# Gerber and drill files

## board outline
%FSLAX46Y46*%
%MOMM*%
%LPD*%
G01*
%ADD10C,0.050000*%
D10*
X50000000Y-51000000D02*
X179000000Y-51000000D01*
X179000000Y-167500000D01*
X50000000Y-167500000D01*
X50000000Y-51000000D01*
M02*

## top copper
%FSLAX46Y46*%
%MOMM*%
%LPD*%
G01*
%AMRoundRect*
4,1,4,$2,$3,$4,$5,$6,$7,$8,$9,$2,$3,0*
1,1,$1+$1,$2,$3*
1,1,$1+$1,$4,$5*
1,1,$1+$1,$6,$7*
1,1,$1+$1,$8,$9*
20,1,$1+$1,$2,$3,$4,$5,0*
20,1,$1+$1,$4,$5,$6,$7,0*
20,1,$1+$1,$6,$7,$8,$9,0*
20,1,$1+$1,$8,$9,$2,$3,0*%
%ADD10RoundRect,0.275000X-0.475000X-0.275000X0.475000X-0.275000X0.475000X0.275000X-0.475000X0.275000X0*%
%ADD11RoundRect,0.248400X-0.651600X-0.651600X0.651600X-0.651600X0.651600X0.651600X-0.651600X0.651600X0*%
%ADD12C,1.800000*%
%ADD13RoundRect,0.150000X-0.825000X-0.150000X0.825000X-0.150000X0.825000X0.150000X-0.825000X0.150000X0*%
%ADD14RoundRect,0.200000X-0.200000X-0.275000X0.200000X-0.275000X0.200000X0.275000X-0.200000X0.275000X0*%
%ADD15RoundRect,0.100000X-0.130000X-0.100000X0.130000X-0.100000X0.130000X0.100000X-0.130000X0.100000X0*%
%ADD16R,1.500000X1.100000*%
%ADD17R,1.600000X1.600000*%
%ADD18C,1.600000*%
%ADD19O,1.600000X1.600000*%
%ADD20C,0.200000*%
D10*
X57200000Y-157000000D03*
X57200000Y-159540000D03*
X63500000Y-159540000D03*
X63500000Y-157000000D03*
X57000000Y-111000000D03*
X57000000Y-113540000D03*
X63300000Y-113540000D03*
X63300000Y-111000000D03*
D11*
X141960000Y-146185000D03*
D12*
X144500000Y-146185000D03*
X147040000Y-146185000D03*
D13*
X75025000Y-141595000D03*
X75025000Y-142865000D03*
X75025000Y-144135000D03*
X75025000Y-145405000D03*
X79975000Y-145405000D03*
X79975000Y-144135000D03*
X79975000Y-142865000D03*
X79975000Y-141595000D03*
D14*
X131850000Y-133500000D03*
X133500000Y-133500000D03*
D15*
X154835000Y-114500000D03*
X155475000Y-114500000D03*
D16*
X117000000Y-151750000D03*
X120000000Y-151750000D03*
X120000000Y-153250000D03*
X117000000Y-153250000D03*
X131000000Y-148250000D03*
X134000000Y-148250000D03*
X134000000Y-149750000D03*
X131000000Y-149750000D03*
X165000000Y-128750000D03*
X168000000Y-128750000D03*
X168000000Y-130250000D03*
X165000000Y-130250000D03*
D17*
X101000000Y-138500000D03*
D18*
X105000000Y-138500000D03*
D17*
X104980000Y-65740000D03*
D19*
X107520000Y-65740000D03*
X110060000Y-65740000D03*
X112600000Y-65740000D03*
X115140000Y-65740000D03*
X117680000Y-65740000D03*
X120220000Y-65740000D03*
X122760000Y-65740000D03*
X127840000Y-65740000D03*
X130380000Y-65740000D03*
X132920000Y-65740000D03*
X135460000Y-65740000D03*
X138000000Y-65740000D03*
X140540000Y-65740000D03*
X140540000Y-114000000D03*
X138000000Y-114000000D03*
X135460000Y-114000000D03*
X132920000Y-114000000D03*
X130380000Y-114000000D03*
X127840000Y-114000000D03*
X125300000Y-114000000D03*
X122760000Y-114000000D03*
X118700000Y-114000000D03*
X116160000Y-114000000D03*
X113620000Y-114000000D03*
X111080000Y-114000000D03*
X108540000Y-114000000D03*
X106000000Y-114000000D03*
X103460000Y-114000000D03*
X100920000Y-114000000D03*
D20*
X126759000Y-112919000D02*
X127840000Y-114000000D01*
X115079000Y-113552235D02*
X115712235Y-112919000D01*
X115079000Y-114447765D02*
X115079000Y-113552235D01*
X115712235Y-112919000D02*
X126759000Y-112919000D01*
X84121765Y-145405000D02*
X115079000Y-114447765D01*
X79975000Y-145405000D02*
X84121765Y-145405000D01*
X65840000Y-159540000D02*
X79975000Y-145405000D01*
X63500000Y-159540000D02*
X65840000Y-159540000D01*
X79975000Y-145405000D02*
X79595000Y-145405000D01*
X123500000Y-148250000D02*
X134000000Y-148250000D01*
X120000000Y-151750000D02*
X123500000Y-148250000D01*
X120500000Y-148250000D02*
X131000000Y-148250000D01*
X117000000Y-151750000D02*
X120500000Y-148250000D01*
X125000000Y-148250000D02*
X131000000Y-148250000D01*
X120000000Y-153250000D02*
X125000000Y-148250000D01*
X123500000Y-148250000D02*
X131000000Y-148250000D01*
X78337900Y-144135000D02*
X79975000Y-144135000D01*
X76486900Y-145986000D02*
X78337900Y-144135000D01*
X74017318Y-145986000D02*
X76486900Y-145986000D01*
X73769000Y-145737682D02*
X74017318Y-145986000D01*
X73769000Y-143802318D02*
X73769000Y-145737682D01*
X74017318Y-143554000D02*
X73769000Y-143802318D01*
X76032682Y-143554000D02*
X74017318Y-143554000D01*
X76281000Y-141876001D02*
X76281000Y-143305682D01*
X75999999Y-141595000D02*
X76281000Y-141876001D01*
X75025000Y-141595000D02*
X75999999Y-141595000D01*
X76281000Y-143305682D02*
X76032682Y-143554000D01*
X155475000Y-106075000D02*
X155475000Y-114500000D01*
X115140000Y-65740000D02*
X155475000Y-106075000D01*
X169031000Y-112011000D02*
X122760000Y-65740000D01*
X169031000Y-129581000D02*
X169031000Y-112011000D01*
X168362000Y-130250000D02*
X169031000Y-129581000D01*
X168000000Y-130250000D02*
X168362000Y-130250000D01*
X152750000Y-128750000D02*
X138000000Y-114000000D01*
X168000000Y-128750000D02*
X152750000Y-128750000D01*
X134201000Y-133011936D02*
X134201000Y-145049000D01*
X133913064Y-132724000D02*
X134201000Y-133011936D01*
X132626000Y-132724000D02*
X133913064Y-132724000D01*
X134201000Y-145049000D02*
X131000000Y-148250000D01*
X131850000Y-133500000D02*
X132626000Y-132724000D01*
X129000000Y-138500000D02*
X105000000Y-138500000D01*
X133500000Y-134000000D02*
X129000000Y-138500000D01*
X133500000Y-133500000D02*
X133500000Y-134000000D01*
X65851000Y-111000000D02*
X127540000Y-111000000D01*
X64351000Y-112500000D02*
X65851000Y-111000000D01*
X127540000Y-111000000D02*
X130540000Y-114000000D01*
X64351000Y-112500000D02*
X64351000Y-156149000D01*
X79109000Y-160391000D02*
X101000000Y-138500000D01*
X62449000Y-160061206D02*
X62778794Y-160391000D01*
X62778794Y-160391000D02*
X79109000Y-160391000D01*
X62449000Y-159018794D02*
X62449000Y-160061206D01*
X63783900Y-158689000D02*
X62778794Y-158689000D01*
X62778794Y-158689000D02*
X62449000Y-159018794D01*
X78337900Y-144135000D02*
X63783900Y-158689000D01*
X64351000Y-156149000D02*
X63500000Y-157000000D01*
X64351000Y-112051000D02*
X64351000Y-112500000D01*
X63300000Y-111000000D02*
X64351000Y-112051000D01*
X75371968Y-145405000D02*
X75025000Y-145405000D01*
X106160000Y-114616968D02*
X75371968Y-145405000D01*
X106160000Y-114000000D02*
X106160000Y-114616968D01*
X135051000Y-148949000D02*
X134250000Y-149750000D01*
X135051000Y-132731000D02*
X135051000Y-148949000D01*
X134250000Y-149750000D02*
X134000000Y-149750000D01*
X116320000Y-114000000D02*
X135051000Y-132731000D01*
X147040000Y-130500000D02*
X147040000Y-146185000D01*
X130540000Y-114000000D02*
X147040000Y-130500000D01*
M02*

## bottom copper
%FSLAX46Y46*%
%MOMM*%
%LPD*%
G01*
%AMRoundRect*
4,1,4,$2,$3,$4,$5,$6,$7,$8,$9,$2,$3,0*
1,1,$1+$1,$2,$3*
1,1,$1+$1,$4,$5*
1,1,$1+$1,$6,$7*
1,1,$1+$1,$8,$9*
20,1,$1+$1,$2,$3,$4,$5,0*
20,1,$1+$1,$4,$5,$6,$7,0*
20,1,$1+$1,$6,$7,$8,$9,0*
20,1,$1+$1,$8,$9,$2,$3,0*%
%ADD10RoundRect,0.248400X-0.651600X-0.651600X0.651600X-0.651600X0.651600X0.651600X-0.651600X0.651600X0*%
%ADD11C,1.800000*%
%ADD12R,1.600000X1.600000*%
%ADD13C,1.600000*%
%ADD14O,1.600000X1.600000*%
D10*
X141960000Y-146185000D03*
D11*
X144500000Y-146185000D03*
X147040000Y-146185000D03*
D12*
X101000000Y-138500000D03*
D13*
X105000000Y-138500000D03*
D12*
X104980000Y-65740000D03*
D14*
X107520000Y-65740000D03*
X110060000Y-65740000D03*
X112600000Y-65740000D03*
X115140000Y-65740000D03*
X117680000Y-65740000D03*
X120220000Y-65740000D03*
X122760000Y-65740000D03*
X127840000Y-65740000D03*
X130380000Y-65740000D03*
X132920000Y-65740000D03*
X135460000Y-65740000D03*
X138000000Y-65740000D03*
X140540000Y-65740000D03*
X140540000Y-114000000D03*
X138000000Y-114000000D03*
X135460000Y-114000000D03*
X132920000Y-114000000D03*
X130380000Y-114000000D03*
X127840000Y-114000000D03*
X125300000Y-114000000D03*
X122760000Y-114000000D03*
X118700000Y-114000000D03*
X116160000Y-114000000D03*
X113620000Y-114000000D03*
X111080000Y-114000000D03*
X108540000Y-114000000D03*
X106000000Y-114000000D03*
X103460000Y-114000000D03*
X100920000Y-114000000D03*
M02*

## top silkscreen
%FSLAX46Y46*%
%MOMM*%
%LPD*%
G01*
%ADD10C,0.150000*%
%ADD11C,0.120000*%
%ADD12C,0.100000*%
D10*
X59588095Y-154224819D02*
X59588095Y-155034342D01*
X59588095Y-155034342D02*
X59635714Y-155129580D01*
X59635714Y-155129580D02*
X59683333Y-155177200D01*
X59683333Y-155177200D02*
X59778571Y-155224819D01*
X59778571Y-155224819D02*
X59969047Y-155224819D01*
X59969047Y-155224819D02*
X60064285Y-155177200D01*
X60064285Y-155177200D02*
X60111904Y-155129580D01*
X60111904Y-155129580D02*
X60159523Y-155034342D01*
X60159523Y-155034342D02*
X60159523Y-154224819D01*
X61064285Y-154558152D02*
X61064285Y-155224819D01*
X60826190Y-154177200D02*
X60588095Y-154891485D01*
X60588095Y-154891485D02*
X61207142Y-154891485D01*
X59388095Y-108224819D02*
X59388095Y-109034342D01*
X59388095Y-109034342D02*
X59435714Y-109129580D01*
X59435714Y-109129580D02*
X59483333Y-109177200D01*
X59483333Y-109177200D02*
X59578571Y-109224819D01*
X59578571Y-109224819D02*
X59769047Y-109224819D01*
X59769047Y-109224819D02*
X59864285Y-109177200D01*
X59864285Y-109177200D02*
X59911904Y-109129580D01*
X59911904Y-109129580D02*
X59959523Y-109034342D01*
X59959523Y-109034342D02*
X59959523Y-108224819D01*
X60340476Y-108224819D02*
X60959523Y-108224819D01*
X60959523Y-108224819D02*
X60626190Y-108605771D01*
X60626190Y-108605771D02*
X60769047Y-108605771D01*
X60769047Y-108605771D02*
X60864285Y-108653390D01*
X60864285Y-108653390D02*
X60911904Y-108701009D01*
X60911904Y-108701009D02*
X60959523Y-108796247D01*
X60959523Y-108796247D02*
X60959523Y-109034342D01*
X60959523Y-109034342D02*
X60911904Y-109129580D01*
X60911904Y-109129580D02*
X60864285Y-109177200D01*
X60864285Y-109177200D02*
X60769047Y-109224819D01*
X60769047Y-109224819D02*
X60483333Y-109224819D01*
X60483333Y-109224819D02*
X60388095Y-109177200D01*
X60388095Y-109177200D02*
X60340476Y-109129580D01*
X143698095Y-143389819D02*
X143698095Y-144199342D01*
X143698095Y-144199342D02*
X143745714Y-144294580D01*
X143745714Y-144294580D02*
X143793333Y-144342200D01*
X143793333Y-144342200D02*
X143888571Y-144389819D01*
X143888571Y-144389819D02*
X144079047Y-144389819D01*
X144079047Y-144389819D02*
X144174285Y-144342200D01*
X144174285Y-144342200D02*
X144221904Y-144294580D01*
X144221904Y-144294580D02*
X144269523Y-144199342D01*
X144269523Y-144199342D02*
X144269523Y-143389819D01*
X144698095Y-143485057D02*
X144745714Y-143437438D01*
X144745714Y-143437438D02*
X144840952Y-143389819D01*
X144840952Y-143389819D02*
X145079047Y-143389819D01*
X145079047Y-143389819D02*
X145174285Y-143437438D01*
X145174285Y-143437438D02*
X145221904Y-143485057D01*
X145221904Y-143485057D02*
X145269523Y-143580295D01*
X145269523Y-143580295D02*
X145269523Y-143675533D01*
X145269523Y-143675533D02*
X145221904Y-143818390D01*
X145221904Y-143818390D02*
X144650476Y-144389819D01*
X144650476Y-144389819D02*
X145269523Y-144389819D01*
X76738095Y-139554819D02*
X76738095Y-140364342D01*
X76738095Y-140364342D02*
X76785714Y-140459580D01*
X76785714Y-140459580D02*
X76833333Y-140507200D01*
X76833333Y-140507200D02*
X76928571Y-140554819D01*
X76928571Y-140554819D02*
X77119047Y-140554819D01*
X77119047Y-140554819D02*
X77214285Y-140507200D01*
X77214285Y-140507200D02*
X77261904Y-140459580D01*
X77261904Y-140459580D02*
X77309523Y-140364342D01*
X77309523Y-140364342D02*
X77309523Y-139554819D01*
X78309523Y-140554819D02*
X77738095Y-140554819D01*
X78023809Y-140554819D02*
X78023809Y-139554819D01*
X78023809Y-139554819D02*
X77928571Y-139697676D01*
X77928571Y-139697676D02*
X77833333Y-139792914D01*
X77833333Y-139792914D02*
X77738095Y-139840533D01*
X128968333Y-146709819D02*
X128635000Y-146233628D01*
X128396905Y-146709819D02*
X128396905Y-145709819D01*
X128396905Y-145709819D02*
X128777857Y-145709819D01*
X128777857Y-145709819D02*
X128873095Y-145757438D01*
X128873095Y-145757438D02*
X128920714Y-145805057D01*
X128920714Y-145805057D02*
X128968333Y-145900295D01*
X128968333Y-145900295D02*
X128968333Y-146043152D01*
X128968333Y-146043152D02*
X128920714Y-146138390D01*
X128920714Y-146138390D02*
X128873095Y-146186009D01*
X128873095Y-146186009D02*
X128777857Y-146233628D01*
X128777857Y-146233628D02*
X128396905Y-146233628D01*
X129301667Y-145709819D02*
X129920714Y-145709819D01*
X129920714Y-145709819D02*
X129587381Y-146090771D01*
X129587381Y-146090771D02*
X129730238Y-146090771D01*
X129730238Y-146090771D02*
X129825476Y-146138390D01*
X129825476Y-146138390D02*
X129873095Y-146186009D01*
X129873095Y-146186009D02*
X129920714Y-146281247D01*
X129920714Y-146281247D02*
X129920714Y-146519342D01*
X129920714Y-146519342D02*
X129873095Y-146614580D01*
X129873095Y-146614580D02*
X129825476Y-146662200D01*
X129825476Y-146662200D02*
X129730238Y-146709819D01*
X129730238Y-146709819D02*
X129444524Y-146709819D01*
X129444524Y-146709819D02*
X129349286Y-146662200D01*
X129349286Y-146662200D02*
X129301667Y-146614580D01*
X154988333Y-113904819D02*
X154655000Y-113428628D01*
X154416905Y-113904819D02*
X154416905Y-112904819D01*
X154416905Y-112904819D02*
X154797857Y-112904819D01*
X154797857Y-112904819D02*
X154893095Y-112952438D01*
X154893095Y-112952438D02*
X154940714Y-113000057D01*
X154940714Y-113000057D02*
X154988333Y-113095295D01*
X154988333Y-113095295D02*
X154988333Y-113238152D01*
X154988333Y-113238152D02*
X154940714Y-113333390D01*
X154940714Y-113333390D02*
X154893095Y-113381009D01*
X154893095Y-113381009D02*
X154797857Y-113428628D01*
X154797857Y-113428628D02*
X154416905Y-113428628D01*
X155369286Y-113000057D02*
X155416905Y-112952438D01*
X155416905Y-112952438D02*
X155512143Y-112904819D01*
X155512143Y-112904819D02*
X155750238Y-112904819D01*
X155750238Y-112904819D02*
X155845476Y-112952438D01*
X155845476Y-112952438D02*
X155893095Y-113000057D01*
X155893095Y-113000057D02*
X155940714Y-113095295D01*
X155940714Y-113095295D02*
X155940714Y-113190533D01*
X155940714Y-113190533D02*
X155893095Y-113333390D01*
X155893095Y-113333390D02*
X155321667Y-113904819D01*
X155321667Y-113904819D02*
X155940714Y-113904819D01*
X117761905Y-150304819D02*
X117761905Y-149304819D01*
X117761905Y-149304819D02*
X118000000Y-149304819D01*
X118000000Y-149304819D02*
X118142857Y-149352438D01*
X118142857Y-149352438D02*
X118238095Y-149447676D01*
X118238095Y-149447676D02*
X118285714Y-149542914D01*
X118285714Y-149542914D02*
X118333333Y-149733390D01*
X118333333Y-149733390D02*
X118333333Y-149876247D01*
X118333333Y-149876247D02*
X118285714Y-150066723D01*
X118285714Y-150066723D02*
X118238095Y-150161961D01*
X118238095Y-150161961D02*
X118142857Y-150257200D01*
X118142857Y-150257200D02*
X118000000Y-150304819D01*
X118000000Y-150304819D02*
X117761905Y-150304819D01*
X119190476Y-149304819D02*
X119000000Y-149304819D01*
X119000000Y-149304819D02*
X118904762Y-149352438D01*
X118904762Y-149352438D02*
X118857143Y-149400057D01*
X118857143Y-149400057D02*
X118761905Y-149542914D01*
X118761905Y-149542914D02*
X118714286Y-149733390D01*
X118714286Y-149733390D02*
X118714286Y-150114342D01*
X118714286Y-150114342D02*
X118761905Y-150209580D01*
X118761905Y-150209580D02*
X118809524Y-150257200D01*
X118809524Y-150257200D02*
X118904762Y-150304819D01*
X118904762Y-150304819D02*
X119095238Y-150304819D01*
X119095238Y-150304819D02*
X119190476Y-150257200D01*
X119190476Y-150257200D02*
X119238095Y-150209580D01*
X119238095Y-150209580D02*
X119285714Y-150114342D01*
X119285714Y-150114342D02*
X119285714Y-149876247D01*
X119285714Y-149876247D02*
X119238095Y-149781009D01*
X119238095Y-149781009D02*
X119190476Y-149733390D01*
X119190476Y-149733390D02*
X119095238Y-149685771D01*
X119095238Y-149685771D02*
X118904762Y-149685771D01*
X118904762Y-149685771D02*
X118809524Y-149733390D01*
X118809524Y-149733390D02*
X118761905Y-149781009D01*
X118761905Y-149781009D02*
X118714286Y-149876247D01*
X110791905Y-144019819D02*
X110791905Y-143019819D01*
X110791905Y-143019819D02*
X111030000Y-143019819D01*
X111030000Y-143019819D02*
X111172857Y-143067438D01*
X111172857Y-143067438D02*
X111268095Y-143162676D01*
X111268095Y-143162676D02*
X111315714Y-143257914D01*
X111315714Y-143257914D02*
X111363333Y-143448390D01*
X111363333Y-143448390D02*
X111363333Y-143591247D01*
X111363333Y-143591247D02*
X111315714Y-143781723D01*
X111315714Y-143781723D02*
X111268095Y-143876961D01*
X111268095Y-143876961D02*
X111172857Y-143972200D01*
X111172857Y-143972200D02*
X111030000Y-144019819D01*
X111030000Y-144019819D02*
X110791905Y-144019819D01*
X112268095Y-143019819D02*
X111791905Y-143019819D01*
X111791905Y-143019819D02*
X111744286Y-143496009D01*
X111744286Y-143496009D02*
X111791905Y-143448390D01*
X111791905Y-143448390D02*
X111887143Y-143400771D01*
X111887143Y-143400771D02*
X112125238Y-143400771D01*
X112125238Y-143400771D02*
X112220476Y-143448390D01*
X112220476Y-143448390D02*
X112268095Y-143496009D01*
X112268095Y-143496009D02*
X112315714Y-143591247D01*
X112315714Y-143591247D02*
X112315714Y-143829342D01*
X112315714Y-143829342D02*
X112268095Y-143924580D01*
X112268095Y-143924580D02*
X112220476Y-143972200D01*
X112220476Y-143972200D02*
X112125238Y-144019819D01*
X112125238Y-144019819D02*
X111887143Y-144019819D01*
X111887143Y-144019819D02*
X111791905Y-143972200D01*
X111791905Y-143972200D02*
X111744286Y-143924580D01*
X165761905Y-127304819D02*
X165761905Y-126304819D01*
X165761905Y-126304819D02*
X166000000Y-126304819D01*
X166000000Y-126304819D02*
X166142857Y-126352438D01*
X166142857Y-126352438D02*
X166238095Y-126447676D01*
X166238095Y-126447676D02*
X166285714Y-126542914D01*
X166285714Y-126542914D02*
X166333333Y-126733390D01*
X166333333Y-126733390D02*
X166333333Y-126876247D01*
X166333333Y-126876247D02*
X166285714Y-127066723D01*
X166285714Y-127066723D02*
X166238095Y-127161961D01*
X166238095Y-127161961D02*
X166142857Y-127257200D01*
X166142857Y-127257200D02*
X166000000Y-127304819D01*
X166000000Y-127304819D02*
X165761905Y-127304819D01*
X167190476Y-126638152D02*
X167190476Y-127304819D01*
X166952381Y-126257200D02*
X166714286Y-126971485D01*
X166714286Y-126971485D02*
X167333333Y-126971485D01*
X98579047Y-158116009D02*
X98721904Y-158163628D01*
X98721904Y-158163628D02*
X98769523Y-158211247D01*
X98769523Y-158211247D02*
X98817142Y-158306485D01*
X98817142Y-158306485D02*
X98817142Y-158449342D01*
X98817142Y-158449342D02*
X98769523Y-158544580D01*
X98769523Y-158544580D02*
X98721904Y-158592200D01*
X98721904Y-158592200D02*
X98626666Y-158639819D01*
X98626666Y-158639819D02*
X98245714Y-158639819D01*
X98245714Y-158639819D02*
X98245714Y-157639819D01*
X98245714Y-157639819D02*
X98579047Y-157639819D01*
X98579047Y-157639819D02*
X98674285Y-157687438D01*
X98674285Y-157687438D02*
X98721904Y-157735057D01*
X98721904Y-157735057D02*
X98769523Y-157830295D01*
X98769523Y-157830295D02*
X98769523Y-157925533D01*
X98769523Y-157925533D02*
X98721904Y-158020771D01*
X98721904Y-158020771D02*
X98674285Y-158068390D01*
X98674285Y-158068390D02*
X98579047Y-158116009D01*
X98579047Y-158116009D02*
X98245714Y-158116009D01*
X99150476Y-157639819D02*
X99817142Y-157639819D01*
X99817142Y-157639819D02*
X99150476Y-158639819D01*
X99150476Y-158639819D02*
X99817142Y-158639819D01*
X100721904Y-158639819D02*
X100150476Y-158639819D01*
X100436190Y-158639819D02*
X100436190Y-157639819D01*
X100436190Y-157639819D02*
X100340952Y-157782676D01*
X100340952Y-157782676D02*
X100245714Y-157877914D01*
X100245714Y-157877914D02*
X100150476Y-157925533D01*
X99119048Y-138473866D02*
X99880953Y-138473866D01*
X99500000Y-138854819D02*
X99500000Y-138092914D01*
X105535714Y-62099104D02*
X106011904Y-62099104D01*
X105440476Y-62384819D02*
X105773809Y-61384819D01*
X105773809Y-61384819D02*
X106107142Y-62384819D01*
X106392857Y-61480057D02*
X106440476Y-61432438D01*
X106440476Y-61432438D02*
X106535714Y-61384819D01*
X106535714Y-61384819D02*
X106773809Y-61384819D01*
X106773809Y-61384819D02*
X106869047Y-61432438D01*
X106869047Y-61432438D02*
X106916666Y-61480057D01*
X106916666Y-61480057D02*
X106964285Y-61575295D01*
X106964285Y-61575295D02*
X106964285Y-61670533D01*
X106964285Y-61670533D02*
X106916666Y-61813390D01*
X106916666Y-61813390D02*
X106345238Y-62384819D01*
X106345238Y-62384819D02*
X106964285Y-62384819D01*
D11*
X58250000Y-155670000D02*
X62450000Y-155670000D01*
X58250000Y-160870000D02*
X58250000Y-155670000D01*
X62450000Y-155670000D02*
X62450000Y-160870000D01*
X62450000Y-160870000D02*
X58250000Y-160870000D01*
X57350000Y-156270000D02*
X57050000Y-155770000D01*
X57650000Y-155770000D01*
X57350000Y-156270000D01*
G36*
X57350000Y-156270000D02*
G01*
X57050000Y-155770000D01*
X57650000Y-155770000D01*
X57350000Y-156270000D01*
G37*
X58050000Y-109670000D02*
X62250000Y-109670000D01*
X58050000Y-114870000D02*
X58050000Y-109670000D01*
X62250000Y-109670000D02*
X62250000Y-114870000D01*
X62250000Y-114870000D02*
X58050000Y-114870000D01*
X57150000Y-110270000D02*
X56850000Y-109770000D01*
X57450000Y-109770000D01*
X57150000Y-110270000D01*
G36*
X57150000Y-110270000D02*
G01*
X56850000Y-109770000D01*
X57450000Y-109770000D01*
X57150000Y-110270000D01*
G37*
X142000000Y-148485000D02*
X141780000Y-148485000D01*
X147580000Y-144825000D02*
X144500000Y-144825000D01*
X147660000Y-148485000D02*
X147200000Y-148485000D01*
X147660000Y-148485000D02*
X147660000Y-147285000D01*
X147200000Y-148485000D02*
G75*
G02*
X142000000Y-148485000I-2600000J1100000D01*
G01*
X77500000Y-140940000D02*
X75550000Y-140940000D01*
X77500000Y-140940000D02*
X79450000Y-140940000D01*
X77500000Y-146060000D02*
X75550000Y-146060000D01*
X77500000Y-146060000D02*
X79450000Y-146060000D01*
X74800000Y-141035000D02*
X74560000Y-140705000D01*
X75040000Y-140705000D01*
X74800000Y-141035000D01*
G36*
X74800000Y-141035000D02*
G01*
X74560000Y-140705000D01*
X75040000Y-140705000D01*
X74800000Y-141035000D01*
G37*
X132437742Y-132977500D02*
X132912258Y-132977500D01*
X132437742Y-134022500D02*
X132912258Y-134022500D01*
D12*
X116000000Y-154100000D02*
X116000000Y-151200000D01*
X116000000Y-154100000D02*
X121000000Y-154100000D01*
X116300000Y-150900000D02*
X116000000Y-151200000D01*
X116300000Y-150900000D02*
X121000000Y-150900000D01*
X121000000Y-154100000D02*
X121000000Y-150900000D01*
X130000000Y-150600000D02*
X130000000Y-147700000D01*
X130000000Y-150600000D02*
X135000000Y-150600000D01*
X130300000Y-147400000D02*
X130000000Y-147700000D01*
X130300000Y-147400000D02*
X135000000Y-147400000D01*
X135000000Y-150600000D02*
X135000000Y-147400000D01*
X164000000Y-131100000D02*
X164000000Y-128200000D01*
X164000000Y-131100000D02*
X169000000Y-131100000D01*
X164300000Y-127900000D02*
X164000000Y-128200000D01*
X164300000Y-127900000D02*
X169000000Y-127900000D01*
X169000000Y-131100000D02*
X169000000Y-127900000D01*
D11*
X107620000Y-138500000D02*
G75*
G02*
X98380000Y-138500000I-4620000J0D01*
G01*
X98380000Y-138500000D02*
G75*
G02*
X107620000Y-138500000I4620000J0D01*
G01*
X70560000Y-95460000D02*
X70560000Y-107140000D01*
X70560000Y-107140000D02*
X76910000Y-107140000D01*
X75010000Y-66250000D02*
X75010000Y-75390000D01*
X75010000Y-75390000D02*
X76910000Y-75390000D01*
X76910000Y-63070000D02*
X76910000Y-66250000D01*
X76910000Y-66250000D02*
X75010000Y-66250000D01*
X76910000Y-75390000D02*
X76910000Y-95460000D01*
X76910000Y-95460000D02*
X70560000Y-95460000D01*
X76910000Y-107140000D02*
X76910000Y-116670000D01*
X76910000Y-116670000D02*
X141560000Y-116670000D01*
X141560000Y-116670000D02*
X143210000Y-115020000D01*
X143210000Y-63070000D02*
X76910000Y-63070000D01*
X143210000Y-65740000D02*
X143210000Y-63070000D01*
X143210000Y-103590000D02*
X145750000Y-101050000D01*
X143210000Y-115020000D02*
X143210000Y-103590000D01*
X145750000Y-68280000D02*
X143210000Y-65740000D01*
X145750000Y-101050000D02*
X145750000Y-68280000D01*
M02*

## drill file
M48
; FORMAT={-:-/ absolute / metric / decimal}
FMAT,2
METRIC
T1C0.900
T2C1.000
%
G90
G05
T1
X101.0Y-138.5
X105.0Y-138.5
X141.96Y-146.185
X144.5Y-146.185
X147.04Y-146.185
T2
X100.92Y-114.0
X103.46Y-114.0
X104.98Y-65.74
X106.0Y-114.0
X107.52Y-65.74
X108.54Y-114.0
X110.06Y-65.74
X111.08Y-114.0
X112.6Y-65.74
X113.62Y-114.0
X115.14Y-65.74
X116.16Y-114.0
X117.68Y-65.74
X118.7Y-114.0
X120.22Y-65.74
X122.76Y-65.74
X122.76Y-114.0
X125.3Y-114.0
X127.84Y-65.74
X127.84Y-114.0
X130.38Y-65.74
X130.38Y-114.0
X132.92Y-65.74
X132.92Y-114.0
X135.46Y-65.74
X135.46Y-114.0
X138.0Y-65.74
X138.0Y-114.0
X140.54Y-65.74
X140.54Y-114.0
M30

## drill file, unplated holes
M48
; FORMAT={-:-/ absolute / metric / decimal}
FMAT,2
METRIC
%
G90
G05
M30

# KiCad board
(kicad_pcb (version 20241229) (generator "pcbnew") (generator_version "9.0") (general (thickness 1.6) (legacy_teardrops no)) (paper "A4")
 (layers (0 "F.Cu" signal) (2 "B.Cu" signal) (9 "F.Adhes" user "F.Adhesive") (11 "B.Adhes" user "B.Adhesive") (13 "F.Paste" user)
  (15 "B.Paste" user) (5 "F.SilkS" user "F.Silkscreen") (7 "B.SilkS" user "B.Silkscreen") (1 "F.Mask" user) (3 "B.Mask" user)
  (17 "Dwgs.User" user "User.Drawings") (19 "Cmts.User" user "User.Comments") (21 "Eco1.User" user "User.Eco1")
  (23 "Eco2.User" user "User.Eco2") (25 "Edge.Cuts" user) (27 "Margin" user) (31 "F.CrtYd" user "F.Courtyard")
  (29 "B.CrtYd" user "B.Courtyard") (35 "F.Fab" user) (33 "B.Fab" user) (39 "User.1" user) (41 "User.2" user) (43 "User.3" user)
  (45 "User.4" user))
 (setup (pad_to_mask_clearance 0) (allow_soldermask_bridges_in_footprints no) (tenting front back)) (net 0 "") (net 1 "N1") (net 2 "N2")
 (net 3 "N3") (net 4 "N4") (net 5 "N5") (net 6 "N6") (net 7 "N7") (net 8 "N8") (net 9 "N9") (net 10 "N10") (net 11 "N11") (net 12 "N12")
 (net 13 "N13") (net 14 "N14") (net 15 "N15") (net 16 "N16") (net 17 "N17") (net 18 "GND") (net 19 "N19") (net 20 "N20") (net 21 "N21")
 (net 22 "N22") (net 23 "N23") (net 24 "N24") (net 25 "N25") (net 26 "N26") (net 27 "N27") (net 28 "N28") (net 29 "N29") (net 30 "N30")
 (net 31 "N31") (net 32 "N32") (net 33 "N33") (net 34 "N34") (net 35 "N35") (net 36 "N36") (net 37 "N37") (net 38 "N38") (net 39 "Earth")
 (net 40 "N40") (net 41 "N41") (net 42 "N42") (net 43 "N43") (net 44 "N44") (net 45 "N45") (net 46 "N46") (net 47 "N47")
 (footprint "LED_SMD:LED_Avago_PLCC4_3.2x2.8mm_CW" (layer "F.Cu") (at 118.5 152.5)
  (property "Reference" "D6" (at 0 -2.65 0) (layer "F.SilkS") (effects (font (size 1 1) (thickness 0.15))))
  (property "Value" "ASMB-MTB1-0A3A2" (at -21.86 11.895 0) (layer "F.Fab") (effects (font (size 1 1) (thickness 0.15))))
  (fp_line (start -2.5 1.6) (end -2.5 -1.3) (stroke (width 0.1) (type solid)) (layer "F.SilkS"))
  (fp_line (start -2.5 1.6) (end 2.5 1.6) (stroke (width 0.1) (type solid)) (layer "F.SilkS"))
  (fp_line (start -2.2 -1.6) (end -2.5 -1.3) (stroke (width 0.1) (type default)) (layer "F.SilkS"))
  (fp_line (start -2.2 -1.6) (end 2.5 -1.6) (stroke (width 0.1) (type solid)) (layer "F.SilkS"))
  (fp_line (start 2.5 1.6) (end 2.5 -1.6) (stroke (width 0.1) (type solid)) (layer "F.SilkS"))
  (pad "1" smd rect (at -1.5 -0.75) (size 1.5 1.1) (layers "F.Cu" "F.Mask" "F.Paste") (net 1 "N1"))
  (pad "2" smd rect (at 1.5 -0.75) (size 1.5 1.1) (layers "F.Cu" "F.Mask" "F.Paste") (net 1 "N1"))
  (pad "3" smd rect (at 1.5 0.75) (size 1.5 1.1) (layers "F.Cu" "F.Mask" "F.Paste") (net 1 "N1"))
  (pad "4" smd rect (at -1.5 0.75) (size 1.5 1.1) (layers "F.Cu" "F.Mask" "F.Paste") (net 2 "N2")))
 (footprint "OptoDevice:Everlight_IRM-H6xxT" (layer "F.Cu") (at 60.35 158.27)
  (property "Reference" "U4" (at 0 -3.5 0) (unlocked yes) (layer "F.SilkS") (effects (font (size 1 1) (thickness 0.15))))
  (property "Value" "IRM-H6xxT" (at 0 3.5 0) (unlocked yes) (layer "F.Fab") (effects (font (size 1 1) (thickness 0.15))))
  (fp_line (start -2.1 -2.6) (end 2.1 -2.6) (stroke (width 0.12) (type default)) (layer "F.SilkS"))
  (fp_line (start -2.1 2.6) (end -2.1 -2.6) (stroke (width 0.12) (type default)) (layer "F.SilkS"))
  (fp_line (start 2.1 -2.6) (end 2.1 2.6) (stroke (width 0.12) (type default)) (layer "F.SilkS"))
  (fp_line (start 2.1 2.6) (end -2.1 2.6) (stroke (width 0.12) (type default)) (layer "F.SilkS"))
  (fp_poly (pts (xy -3.3 -2.5) (xy -2.7 -2.5) (xy -3 -2)) (stroke (width 0.12) (type solid)) (fill yes) (layer "F.SilkS"))
  (pad "1" smd roundrect (at -3.15 -1.27) (size 1.5 1.1) (layers "F.Cu" "F.Mask" "F.Paste") (roundrect_rratio 0.25) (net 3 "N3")
   (thermal_bridge_angle 45))
  (pad "2" smd roundrect (at -3.15 1.27) (size 1.5 1.1) (layers "F.Cu" "F.Mask" "F.Paste") (roundrect_rratio 0.25) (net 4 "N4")
   (thermal_bridge_angle 45))
  (pad "3" smd roundrect (at 3.15 1.27) (size 1.5 1.1) (layers "F.Cu" "F.Mask" "F.Paste") (roundrect_rratio 0.25) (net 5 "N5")
   (thermal_bridge_angle 45))
  (pad "4" smd roundrect (at 3.15 -1.27) (size 1.5 1.1) (layers "F.Cu" "F.Mask" "F.Paste") (roundrect_rratio 0.25) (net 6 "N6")
   (thermal_bridge_angle 45)))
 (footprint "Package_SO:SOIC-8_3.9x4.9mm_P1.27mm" (layer "F.Cu") (at 77.5 143.5)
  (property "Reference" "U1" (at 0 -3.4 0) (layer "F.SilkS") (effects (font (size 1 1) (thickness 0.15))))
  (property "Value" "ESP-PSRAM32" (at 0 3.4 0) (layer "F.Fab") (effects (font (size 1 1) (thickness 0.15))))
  (fp_line (start 0 -2.56) (end -1.95 -2.56) (stroke (width 0.12) (type solid)) (layer "F.SilkS"))
  (fp_line (start 0 -2.56) (end 1.95 -2.56) (stroke (width 0.12) (type solid)) (layer "F.SilkS"))
  (fp_line (start 0 2.56) (end -1.95 2.56) (stroke (width 0.12) (type solid)) (layer "F.SilkS"))
  (fp_line (start 0 2.56) (end 1.95 2.56) (stroke (width 0.12) (type solid)) (layer "F.SilkS"))
  (fp_poly
   (pts (xy -2.7 -2.465) (xy -2.94 -2.795) (xy -2.46 -2.795) (xy -2.7 -2.465)) (stroke (width 0.12) (type solid)) (fill yes)
   (layer "F.SilkS"))
  (pad "1" smd roundrect (at -2.475 -1.905) (size 1.95 0.6) (layers "F.Cu" "F.Mask" "F.Paste") (roundrect_rratio 0.25) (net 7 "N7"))
  (pad "2" smd roundrect (at -2.475 -0.635) (size 1.95 0.6) (layers "F.Cu" "F.Mask" "F.Paste") (roundrect_rratio 0.25) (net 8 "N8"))
  (pad "3" smd roundrect (at -2.475 0.635) (size 1.95 0.6) (layers "F.Cu" "F.Mask" "F.Paste") (roundrect_rratio 0.25) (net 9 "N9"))
  (pad "4" smd roundrect (at -2.475 1.905) (size 1.95 0.6) (layers "F.Cu" "F.Mask" "F.Paste") (roundrect_rratio 0.25) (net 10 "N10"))
  (pad "5" smd roundrect (at 2.475 1.905) (size 1.95 0.6) (layers "F.Cu" "F.Mask" "F.Paste") (roundrect_rratio 0.25) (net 5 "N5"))
  (pad "6" smd roundrect (at 2.475 0.635) (size 1.95 0.6) (layers "F.Cu" "F.Mask" "F.Paste") (roundrect_rratio 0.25) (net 7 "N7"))
  (pad "7" smd roundrect (at 2.475 -0.635) (size 1.95 0.6) (layers "F.Cu" "F.Mask" "F.Paste") (roundrect_rratio 0.25) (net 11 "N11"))
  (pad "8" smd roundrect (at 2.475 -1.905) (size 1.95 0.6) (layers "F.Cu" "F.Mask" "F.Paste") (roundrect_rratio 0.25) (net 10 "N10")))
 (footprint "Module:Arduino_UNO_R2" (layer "F.Cu") (at 104.98 65.74)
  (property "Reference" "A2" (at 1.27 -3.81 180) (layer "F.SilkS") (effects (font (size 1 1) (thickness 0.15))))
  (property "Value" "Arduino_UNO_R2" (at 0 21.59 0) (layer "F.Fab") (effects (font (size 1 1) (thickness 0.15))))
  (fp_line (start -34.42 29.72) (end -34.42 41.4) (stroke (width 0.12) (type solid)) (layer "F.SilkS"))
  (fp_line (start -34.42 41.4) (end -28.07 41.4) (stroke (width 0.12) (type solid)) (layer "F.SilkS"))
  (fp_line (start -29.97 0.51) (end -29.97 9.65) (stroke (width 0.12) (type solid)) (layer "F.SilkS"))
  (fp_line (start -29.97 9.65) (end -28.07 9.65) (stroke (width 0.12) (type solid)) (layer "F.SilkS"))
  (fp_line (start -28.07 -2.67) (end -28.07 0.51) (stroke (width 0.12) (type solid)) (layer "F.SilkS"))
  (fp_line (start -28.07 0.51) (end -29.97 0.51) (stroke (width 0.12) (type solid)) (layer "F.SilkS"))
  (fp_line (start -28.07 9.65) (end -28.07 29.72) (stroke (width 0.12) (type solid)) (layer "F.SilkS"))
  (fp_line (start -28.07 29.72) (end -34.42 29.72) (stroke (width 0.12) (type solid)) (layer "F.SilkS"))
  (fp_line (start -28.07 41.4) (end -28.07 50.93) (stroke (width 0.12) (type solid)) (layer "F.SilkS"))
  (fp_line (start -28.07 50.93) (end 36.58 50.93) (stroke (width 0.12) (type solid)) (layer "F.SilkS"))
  (fp_line (start 36.58 50.93) (end 38.23 49.28) (stroke (width 0.12) (type solid)) (layer "F.SilkS"))
  (fp_line (start 38.23 -2.67) (end -28.07 -2.67) (stroke (width 0.12) (type solid)) (layer "F.SilkS"))
  (fp_line (start 38.23 0) (end 38.23 -2.67) (stroke (width 0.12) (type solid)) (layer "F.SilkS"))
  (fp_line (start 38.23 37.85) (end 40.77 35.31) (stroke (width 0.12) (type solid)) (layer "F.SilkS"))
  (fp_line (start 38.23 49.28) (end 38.23 37.85) (stroke (width 0.12) (type solid)) (layer "F.SilkS"))
  (fp_line (start 40.77 2.54) (end 38.23 0) (stroke (width 0.12) (type solid)) (layer "F.SilkS"))
  (fp_line (start 40.77 35.31) (end 40.77 2.54) (stroke (width 0.12) (type solid)) (layer "F.SilkS"))
  (pad "1" thru_hole rect (at 0 0 90) (size 1.6 1.6) (drill 1) (layers "*.Cu" "*.Mask") (remove_unused_layers no) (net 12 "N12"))
  (pad "2" thru_hole oval (at 2.54 0 90) (size 1.6 1.6) (drill 1) (layers "*.Cu" "*.Mask") (remove_unused_layers no) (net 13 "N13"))
  (pad "3" thru_hole oval (at 5.08 0 90) (size 1.6 1.6) (drill 1) (layers "*.Cu" "*.Mask") (remove_unused_layers no) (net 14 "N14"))
  (pad "4" thru_hole oval (at 7.62 0 90) (size 1.6 1.6) (drill 1) (layers "*.Cu" "*.Mask") (remove_unused_layers no) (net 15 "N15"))
  (pad "5" thru_hole oval (at 10.16 0 90) (size 1.6 1.6) (drill 1) (layers "*.Cu" "*.Mask") (remove_unused_layers no) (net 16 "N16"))
  (pad "6" thru_hole oval (at 12.7 0 90) (size 1.6 1.6) (drill 1) (layers "*.Cu" "*.Mask") (remove_unused_layers no) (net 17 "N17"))
  (pad "7" thru_hole oval (at 15.24 0 90) (size 1.6 1.6) (drill 1) (layers "*.Cu" "*.Mask") (remove_unused_layers no) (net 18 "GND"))
  (pad "8" thru_hole oval (at 17.78 0 90) (size 1.6 1.6) (drill 1) (layers "*.Cu" "*.Mask") (remove_unused_layers no) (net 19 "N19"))
  (pad "9" thru_hole oval (at 22.86 0 90) (size 1.6 1.6) (drill 1) (layers "*.Cu" "*.Mask") (remove_unused_layers no) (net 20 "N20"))
  (pad "10" thru_hole oval (at 25.4 0 90) (size 1.6 1.6) (drill 1) (layers "*.Cu" "*.Mask") (remove_unused_layers no) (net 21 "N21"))
  (pad "11" thru_hole oval (at 27.94 0 90) (size 1.6 1.6) (drill 1) (layers "*.Cu" "*.Mask") (remove_unused_layers no) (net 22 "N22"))
  (pad "12" thru_hole oval (at 30.48 0 90) (size 1.6 1.6) (drill 1) (layers "*.Cu" "*.Mask") (remove_unused_layers no) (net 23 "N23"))
  (pad "13" thru_hole oval (at 33.02 0 90) (size 1.6 1.6) (drill 1) (layers "*.Cu" "*.Mask") (remove_unused_layers no) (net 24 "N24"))
  (pad "14" thru_hole oval (at 35.56 0 90) (size 1.6 1.6) (drill 1) (layers "*.Cu" "*.Mask") (remove_unused_layers no) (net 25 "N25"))
  (pad "15" thru_hole oval (at 35.56 48.26 90) (size 1.6 1.6) (drill 1) (layers "*.Cu" "*.Mask") (remove_unused_layers no) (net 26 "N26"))
  (pad "16" thru_hole oval (at 33.02 48.26 90) (size 1.6 1.6) (drill 1) (layers "*.Cu" "*.Mask") (remove_unused_layers no) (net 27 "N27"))
  (pad "17" thru_hole oval (at 30.48 48.26 90) (size 1.6 1.6) (drill 1) (layers "*.Cu" "*.Mask") (remove_unused_layers no) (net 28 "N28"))
  (pad "18" thru_hole oval (at 27.94 48.26 90) (size 1.6 1.6) (drill 1) (layers "*.Cu" "*.Mask") (remove_unused_layers no) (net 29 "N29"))
  (pad "19" thru_hole oval (at 25.4 48.26 90) (size 1.6 1.6) (drill 1) (layers "*.Cu" "*.Mask") (remove_unused_layers no) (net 6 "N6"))
  (pad "20" thru_hole oval (at 22.86 48.26 90) (size 1.6 1.6) (drill 1) (layers "*.Cu" "*.Mask") (remove_unused_layers no) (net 5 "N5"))
  (pad "21" thru_hole oval (at 20.32 48.26 90) (size 1.6 1.6) (drill 1) (layers "*.Cu" "*.Mask") (remove_unused_layers no) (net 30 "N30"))
  (pad "22" thru_hole oval (at 17.78 48.26 90) (size 1.6 1.6) (drill 1) (layers "*.Cu" "*.Mask") (remove_unused_layers no) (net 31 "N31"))
  (pad "23" thru_hole oval (at 13.72 48.26 90) (size 1.6 1.6) (drill 1) (layers "*.Cu" "*.Mask") (remove_unused_layers no) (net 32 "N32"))
  (pad "24" thru_hole oval (at 11.18 48.26 90) (size 1.6 1.6) (drill 1) (layers "*.Cu" "*.Mask") (remove_unused_layers no) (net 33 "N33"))
  (pad "25" thru_hole oval (at 8.64 48.26 90) (size 1.6 1.6) (drill 1) (layers "*.Cu" "*.Mask") (remove_unused_layers no) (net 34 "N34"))
  (pad "26" thru_hole oval (at 6.1 48.26 90) (size 1.6 1.6) (drill 1) (layers "*.Cu" "*.Mask") (remove_unused_layers no) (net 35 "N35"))
  (pad "27" thru_hole oval (at 3.56 48.26 90) (size 1.6 1.6) (drill 1) (layers "*.Cu" "*.Mask") (remove_unused_layers no) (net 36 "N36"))
  (pad "28" thru_hole oval (at 1.02 48.26 90) (size 1.6 1.6) (drill 1) (layers "*.Cu" "*.Mask") (remove_unused_layers no) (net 10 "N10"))
  (pad "29" thru_hole oval (at -1.52 48.26 90) (size 1.6 1.6) (drill 1) (layers "*.Cu" "*.Mask") (remove_unused_layers no) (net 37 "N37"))
  (pad "30" thru_hole oval (at -4.06 48.26 90) (size 1.6 1.6) (drill 1) (layers "*.Cu" "*.Mask") (remove_unused_layers no) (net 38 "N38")))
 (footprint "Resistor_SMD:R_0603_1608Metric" (layer "F.Cu") (at 132.675 133.5)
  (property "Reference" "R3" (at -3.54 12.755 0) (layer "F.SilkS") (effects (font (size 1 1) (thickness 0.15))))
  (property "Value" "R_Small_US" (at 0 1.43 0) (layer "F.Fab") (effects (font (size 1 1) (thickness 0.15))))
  (fp_line (start -0.237258 -0.5225) (end 0.237258 -0.5225) (stroke (width 0.12) (type solid)) (layer "F.SilkS"))
  (fp_line (start -0.237258 0.5225) (end 0.237258 0.5225) (stroke (width 0.12) (type solid)) (layer "F.SilkS"))
  (pad "1" smd roundrect (at -0.825 0) (size 0.8 0.95) (layers "F.Cu" "F.Mask" "F.Paste") (roundrect_rratio 0.25) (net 1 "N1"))
  (pad "2" smd roundrect (at 0.825 0) (size 0.8 0.95) (layers "F.Cu" "F.Mask" "F.Paste") (roundrect_rratio 0.25) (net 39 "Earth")))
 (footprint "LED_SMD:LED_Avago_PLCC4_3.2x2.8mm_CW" (layer "F.Cu") (at 166.5 129.5)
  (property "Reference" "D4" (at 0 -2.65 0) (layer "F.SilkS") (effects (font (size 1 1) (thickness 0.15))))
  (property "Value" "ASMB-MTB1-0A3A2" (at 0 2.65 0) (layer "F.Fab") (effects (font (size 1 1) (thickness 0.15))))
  (fp_line (start -2.5 1.6) (end -2.5 -1.3) (stroke (width 0.1) (type solid)) (layer "F.SilkS"))
  (fp_line (start -2.5 1.6) (end 2.5 1.6) (stroke (width 0.1) (type solid)) (layer "F.SilkS"))
  (fp_line (start -2.2 -1.6) (end -2.5 -1.3) (stroke (width 0.1) (type default)) (layer "F.SilkS"))
  (fp_line (start -2.2 -1.6) (end 2.5 -1.6) (stroke (width 0.1) (type solid)) (layer "F.SilkS"))
  (fp_line (start 2.5 1.6) (end 2.5 -1.6) (stroke (width 0.1) (type solid)) (layer "F.SilkS"))
  (pad "1" smd rect (at -1.5 -0.75) (size 1.5 1.1) (layers "F.Cu" "F.Mask" "F.Paste") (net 27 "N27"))
  (pad "2" smd rect (at 1.5 -0.75) (size 1.5 1.1) (layers "F.Cu" "F.Mask" "F.Paste") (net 27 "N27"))
  (pad "3" smd rect (at 1.5 0.75) (size 1.5 1.1) (layers "F.Cu" "F.Mask" "F.Paste") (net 19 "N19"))
  (pad "4" smd rect (at -1.5 0.75) (size 1.5 1.1) (layers "F.Cu" "F.Mask" "F.Paste") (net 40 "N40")))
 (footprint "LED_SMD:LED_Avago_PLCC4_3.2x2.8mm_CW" (layer "F.Cu") (at 132.5 149)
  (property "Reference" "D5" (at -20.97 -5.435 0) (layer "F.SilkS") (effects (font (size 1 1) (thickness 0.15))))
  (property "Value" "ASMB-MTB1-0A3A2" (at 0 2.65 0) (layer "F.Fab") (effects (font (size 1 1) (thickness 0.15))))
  (fp_line (start -2.5 1.6) (end -2.5 -1.3) (stroke (width 0.1) (type solid)) (layer "F.SilkS"))
  (fp_line (start -2.5 1.6) (end 2.5 1.6) (stroke (width 0.1) (type solid)) (layer "F.SilkS"))
  (fp_line (start -2.2 -1.6) (end -2.5 -1.3) (stroke (width 0.1) (type default)) (layer "F.SilkS"))
  (fp_line (start -2.2 -1.6) (end 2.5 -1.6) (stroke (width 0.1) (type solid)) (layer "F.SilkS"))
  (fp_line (start 2.5 1.6) (end 2.5 -1.6) (stroke (width 0.1) (type solid)) (layer "F.SilkS"))
  (pad "1" smd rect (at -1.5 -0.75) (size 1.5 1.1) (layers "F.Cu" "F.Mask" "F.Paste") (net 1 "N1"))
  (pad "2" smd rect (at 1.5 -0.75) (size 1.5 1.1) (layers "F.Cu" "F.Mask" "F.Paste") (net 1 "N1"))
  (pad "3" smd rect (at 1.5 0.75) (size 1.5 1.1) (layers "F.Cu" "F.Mask" "F.Paste") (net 33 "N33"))
  (pad "4" smd rect (at -1.5 0.75) (size 1.5 1.1) (layers "F.Cu" "F.Mask" "F.Paste") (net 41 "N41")))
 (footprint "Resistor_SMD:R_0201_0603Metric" (layer "F.Cu") (at 155.155 114.5)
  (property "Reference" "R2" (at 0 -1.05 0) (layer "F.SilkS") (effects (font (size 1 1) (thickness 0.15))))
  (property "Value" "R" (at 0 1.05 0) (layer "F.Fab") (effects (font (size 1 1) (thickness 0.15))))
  (pad "" smd roundrect (at -0.345 0) (size 0.318 0.36) (layers "F.Paste") (roundrect_rratio 0.25))
  (pad "" smd roundrect (at 0.345 0) (size 0.318 0.36) (layers "F.Paste") (roundrect_rratio 0.25))
  (pad "1" smd roundrect (at -0.32 0) (size 0.46 0.4) (layers "F.Cu" "F.Mask") (roundrect_rratio 0.25) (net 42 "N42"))
  (pad "2" smd roundrect (at 0.32 0) (size 0.46 0.4) (layers "F.Cu" "F.Mask") (roundrect_rratio 0.25) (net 16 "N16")))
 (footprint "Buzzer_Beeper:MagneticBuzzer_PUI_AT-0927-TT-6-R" (layer "F.Cu") (at 101 138.5)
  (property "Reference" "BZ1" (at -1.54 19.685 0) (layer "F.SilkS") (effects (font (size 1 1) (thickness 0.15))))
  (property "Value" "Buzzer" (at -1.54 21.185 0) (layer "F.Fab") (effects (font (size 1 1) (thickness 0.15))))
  (fp_circle (center 2 0) (end 6.62 0) (stroke (width 0.12) (type solid)) (fill no) (layer "F.SilkS"))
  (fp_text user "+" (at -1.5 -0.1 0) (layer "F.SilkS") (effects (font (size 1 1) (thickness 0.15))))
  (pad "1" thru_hole rect (at 0 0) (size 1.6 1.6) (drill 0.9) (layers "*.Cu" "*.Mask") (remove_unused_layers no) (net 7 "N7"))
  (pad "2" thru_hole circle (at 4 0) (size 1.6 1.6) (drill 0.9) (layers "*.Cu" "*.Mask") (remove_unused_layers no) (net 39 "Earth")))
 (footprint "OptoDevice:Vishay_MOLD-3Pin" (layer "F.Cu") (at 141.96 146.185)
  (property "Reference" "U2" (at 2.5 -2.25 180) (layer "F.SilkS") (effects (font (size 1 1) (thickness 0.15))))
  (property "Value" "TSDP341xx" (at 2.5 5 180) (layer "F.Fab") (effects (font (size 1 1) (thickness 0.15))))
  (fp_line (start 0.04 2.3) (end -0.18 2.3) (stroke (width 0.12) (type solid)) (layer "F.SilkS"))
  (fp_line (start 5.62 -1.36) (end 2.54 -1.36) (stroke (width 0.12) (type solid)) (layer "F.SilkS"))
  (fp_line (start 5.7 2.3) (end 5.24 2.3) (stroke (width 0.12) (type solid)) (layer "F.SilkS"))
  (fp_line (start 5.7 2.3) (end 5.7 1.1) (stroke (width 0.12) (type solid)) (layer "F.SilkS"))
  (fp_arc (start 5.24 2.3) (mid 2.64 4.023119) (end 0.04 2.3) (stroke (width 0.12) (type solid)) (layer "F.SilkS"))
  (pad "1" thru_hole roundrect (at 0 0) (size 1.8 1.8) (drill 0.9) (layers "*.Cu" "*.Mask") (remove_unused_layers no)
   (roundrect_rratio 0.138) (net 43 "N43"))
  (pad "2" thru_hole circle (at 2.54 0) (size 1.8 1.8) (drill 0.9) (layers "*.Cu" "*.Mask") (remove_unused_layers no) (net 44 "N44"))
  (pad "3" thru_hole circle (at 5.08 0) (size 1.8 1.8) (drill 0.9) (layers "*.Cu" "*.Mask") (remove_unused_layers no) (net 6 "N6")))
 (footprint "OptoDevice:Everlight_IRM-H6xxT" (layer "F.Cu") (at 60.15 112.27)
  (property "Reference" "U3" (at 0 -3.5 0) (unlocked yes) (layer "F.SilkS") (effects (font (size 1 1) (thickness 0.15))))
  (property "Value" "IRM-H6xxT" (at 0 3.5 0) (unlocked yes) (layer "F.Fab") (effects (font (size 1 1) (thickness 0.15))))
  (fp_line (start -2.1 -2.6) (end 2.1 -2.6) (stroke (width 0.12) (type default)) (layer "F.SilkS"))
  (fp_line (start -2.1 2.6) (end -2.1 -2.6) (stroke (width 0.12) (type default)) (layer "F.SilkS"))
  (fp_line (start 2.1 -2.6) (end 2.1 2.6) (stroke (width 0.12) (type default)) (layer "F.SilkS"))
  (fp_line (start 2.1 2.6) (end -2.1 2.6) (stroke (width 0.12) (type default)) (layer "F.SilkS"))
  (fp_poly (pts (xy -3.3 -2.5) (xy -2.7 -2.5) (xy -3 -2)) (stroke (width 0.12) (type solid)) (fill yes) (layer "F.SilkS"))
  (pad "1" smd roundrect (at -3.15 -1.27) (size 1.5 1.1) (layers "F.Cu" "F.Mask" "F.Paste") (roundrect_rratio 0.25) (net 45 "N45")
   (thermal_bridge_angle 45))
  (pad "2" smd roundrect (at -3.15 1.27) (size 1.5 1.1) (layers "F.Cu" "F.Mask" "F.Paste") (roundrect_rratio 0.25) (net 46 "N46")
   (thermal_bridge_angle 45))
  (pad "3" smd roundrect (at 3.15 1.27) (size 1.5 1.1) (layers "F.Cu" "F.Mask" "F.Paste") (roundrect_rratio 0.25) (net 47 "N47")
   (thermal_bridge_angle 45))
  (pad "4" smd roundrect (at 3.15 -1.27) (size 1.5 1.1) (layers "F.Cu" "F.Mask" "F.Paste") (roundrect_rratio 0.25) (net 6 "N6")
   (thermal_bridge_angle 45)))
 (gr_rect (start 50 51) (end 179 167.5) (stroke (width 0.05) (type default)) (fill no) (layer "Edge.Cuts"))
 (segment (start 64.351 112.5) (end 65.851 111) (width 0.2) (layer "F.Cu") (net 6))
 (segment (start 147.04 130.5) (end 147.04 146.185) (width 0.2) (layer "F.Cu") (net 6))
 (segment (start 64.351 156.149) (end 63.5 157) (width 0.2) (layer "F.Cu") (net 6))
 (segment (start 127.54 111) (end 130.54 114) (width 0.2) (layer "F.Cu") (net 6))
 (segment (start 63.3 111) (end 64.351 112.051) (width 0.2) (layer "F.Cu") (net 6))
 (segment (start 130.54 114) (end 147.04 130.5) (width 0.2) (layer "F.Cu") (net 6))
 (segment (start 64.351 112.5) (end 64.351 156.149) (width 0.2) (layer "F.Cu") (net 6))
 (segment (start 64.351 112.051) (end 64.351 112.5) (width 0.2) (layer "F.Cu") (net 6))
 (segment (start 65.851 111) (end 127.54 111) (width 0.2) (layer "F.Cu") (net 6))
 (segment (start 169.031 112.011) (end 122.76 65.74) (width 0.2) (layer "F.Cu") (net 19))
 (segment (start 168.362 130.25) (end 169.031 129.581) (width 0.2) (layer "F.Cu") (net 19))
 (segment (start 169.031 129.581) (end 169.031 112.011) (width 0.2) (layer "F.Cu") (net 19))
 (segment (start 168 130.25) (end 168.362 130.25) (width 0.2) (layer "F.Cu") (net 19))
 (segment (start 65.84 159.54) (end 79.975 145.405) (width 0.2) (layer "F.Cu") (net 5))
 (segment (start 63.5 159.54) (end 65.84 159.54) (width 0.2) (layer "F.Cu") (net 5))
 (segment (start 79.975 145.405) (end 79.595 145.405) (width 0.2) (layer "F.Cu") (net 5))
 (segment (start 115.079 114.447765) (end 115.079 113.552235) (width 0.2) (layer "F.Cu") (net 5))
 (segment (start 126.759 112.919) (end 127.84 114) (width 0.2) (layer "F.Cu") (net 5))
 (segment (start 79.975 145.405) (end 84.121765 145.405) (width 0.2) (layer "F.Cu") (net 5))
 (segment (start 115.079 113.552235) (end 115.712235 112.919) (width 0.2) (layer "F.Cu") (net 5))
 (segment (start 115.712235 112.919) (end 126.759 112.919) (width 0.2) (layer "F.Cu") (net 5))
 (segment (start 84.121765 145.405) (end 115.079 114.447765) (width 0.2) (layer "F.Cu") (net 5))
 (segment (start 106.16 114) (end 106.16 114.616968) (width 0.2) (layer "F.Cu") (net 10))
 (segment (start 75.371968 145.405) (end 75.025 145.405) (width 0.2) (layer "F.Cu") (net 10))
 (segment (start 106.16 114.616968) (end 75.371968 145.405) (width 0.2) (layer "F.Cu") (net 10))
 (segment (start 135.051 132.731) (end 135.051 148.949) (width 0.2) (layer "F.Cu") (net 33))
 (segment (start 134.25 149.75) (end 134 149.75) (width 0.2) (layer "F.Cu") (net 33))
 (segment (start 135.051 148.949) (end 134.25 149.75) (width 0.2) (layer "F.Cu") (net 33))
 (segment (start 116.32 114) (end 135.051 132.731) (width 0.2) (layer "F.Cu") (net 33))
 (segment (start 152.75 128.75) (end 138 114) (width 0.2) (layer "F.Cu") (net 27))
 (segment (start 168 128.75) (end 152.75 128.75) (width 0.2) (layer "F.Cu") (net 27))
 (segment (start 155.475 106.075) (end 155.475 114.5) (width 0.2) (layer "F.Cu") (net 16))
 (segment (start 115.14 65.74) (end 155.475 106.075) (width 0.2) (layer "F.Cu") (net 16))
 (segment (start 76.4869 145.986) (end 78.3379 144.135) (width 0.2) (layer "F.Cu") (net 7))
 (segment (start 74.017318 145.986) (end 76.4869 145.986) (width 0.2) (layer "F.Cu") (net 7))
 (segment (start 74.017318 143.554) (end 73.769 143.802318) (width 0.2) (layer "F.Cu") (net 7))
 (segment (start 78.3379 144.135) (end 63.7839 158.689) (width 0.2) (layer "F.Cu") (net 7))
 (segment (start 76.032682 143.554) (end 74.017318 143.554) (width 0.2) (layer "F.Cu") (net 7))
 (segment (start 73.769 143.802318) (end 73.769 145.737682) (width 0.2) (layer "F.Cu") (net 7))
 (segment (start 63.7839 158.689) (end 62.778794 158.689) (width 0.2) (layer "F.Cu") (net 7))
 (segment (start 62.449 160.061206) (end 62.778794 160.391) (width 0.2) (layer "F.Cu") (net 7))
 (segment (start 78.3379 144.135) (end 79.975 144.135) (width 0.2) (layer "F.Cu") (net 7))
 (segment (start 79.109 160.391) (end 101 138.5) (width 0.2) (layer "F.Cu") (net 7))
 (segment (start 62.778794 158.689) (end 62.449 159.018794) (width 0.2) (layer "F.Cu") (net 7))
 (segment (start 62.449 159.018794) (end 62.449 160.061206) (width 0.2) (layer "F.Cu") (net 7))
 (segment (start 62.778794 160.391) (end 79.109 160.391) (width 0.2) (layer "F.Cu") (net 7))
 (segment (start 75.025 141.595) (end 75.999999 141.595) (width 0.2) (layer "F.Cu") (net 7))
 (segment (start 76.281 141.876001) (end 76.281 143.305682) (width 0.2) (layer "F.Cu") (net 7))
 (segment (start 73.769 145.737682) (end 74.017318 145.986) (width 0.2) (layer "F.Cu") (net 7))
 (segment (start 75.999999 141.595) (end 76.281 141.876001) (width 0.2) (layer "F.Cu") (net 7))
 (segment (start 76.281 143.305682) (end 76.032682 143.554) (width 0.2) (layer "F.Cu") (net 7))
 (segment (start 133.5 134) (end 129 138.5) (width 0.2) (layer "F.Cu") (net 39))
 (segment (start 129 138.5) (end 105 138.5) (width 0.2) (layer "F.Cu") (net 39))
 (segment (start 133.5 133.5) (end 133.5 134) (width 0.2) (layer "F.Cu") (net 39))
 (segment (start 131.85 133.5) (end 132.626 132.724) (width 0.2) (layer "F.Cu") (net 1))
 (segment (start 125 148.25) (end 131 148.25) (width 0.2) (layer "F.Cu") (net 1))
 (segment (start 117 151.75) (end 120.5 148.25) (width 0.2) (layer "F.Cu") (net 1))
 (segment (start 134.201 133.011936) (end 134.201 145.049) (width 0.2) (layer "F.Cu") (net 1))
 (segment (start 134.201 145.049) (end 131 148.25) (width 0.2) (layer "F.Cu") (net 1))
 (segment (start 123.5 148.25) (end 131 148.25) (width 0.2) (layer "F.Cu") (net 1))
 (segment (start 120 153.25) (end 125 148.25) (width 0.2) (layer "F.Cu") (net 1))
 (segment (start 120.5 148.25) (end 131 148.25) (width 0.2) (layer "F.Cu") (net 1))
 (segment (start 123.5 148.25) (end 134 148.25) (width 0.2) (layer "F.Cu") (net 1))
 (segment (start 133.913064 132.724) (end 134.201 133.011936) (width 0.2) (layer "F.Cu") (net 1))
 (segment (start 120 151.75) (end 123.5 148.25) (width 0.2) (layer "F.Cu") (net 1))
 (segment (start 132.626 132.724) (end 133.913064 132.724) (width 0.2) (layer "F.Cu") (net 1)))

